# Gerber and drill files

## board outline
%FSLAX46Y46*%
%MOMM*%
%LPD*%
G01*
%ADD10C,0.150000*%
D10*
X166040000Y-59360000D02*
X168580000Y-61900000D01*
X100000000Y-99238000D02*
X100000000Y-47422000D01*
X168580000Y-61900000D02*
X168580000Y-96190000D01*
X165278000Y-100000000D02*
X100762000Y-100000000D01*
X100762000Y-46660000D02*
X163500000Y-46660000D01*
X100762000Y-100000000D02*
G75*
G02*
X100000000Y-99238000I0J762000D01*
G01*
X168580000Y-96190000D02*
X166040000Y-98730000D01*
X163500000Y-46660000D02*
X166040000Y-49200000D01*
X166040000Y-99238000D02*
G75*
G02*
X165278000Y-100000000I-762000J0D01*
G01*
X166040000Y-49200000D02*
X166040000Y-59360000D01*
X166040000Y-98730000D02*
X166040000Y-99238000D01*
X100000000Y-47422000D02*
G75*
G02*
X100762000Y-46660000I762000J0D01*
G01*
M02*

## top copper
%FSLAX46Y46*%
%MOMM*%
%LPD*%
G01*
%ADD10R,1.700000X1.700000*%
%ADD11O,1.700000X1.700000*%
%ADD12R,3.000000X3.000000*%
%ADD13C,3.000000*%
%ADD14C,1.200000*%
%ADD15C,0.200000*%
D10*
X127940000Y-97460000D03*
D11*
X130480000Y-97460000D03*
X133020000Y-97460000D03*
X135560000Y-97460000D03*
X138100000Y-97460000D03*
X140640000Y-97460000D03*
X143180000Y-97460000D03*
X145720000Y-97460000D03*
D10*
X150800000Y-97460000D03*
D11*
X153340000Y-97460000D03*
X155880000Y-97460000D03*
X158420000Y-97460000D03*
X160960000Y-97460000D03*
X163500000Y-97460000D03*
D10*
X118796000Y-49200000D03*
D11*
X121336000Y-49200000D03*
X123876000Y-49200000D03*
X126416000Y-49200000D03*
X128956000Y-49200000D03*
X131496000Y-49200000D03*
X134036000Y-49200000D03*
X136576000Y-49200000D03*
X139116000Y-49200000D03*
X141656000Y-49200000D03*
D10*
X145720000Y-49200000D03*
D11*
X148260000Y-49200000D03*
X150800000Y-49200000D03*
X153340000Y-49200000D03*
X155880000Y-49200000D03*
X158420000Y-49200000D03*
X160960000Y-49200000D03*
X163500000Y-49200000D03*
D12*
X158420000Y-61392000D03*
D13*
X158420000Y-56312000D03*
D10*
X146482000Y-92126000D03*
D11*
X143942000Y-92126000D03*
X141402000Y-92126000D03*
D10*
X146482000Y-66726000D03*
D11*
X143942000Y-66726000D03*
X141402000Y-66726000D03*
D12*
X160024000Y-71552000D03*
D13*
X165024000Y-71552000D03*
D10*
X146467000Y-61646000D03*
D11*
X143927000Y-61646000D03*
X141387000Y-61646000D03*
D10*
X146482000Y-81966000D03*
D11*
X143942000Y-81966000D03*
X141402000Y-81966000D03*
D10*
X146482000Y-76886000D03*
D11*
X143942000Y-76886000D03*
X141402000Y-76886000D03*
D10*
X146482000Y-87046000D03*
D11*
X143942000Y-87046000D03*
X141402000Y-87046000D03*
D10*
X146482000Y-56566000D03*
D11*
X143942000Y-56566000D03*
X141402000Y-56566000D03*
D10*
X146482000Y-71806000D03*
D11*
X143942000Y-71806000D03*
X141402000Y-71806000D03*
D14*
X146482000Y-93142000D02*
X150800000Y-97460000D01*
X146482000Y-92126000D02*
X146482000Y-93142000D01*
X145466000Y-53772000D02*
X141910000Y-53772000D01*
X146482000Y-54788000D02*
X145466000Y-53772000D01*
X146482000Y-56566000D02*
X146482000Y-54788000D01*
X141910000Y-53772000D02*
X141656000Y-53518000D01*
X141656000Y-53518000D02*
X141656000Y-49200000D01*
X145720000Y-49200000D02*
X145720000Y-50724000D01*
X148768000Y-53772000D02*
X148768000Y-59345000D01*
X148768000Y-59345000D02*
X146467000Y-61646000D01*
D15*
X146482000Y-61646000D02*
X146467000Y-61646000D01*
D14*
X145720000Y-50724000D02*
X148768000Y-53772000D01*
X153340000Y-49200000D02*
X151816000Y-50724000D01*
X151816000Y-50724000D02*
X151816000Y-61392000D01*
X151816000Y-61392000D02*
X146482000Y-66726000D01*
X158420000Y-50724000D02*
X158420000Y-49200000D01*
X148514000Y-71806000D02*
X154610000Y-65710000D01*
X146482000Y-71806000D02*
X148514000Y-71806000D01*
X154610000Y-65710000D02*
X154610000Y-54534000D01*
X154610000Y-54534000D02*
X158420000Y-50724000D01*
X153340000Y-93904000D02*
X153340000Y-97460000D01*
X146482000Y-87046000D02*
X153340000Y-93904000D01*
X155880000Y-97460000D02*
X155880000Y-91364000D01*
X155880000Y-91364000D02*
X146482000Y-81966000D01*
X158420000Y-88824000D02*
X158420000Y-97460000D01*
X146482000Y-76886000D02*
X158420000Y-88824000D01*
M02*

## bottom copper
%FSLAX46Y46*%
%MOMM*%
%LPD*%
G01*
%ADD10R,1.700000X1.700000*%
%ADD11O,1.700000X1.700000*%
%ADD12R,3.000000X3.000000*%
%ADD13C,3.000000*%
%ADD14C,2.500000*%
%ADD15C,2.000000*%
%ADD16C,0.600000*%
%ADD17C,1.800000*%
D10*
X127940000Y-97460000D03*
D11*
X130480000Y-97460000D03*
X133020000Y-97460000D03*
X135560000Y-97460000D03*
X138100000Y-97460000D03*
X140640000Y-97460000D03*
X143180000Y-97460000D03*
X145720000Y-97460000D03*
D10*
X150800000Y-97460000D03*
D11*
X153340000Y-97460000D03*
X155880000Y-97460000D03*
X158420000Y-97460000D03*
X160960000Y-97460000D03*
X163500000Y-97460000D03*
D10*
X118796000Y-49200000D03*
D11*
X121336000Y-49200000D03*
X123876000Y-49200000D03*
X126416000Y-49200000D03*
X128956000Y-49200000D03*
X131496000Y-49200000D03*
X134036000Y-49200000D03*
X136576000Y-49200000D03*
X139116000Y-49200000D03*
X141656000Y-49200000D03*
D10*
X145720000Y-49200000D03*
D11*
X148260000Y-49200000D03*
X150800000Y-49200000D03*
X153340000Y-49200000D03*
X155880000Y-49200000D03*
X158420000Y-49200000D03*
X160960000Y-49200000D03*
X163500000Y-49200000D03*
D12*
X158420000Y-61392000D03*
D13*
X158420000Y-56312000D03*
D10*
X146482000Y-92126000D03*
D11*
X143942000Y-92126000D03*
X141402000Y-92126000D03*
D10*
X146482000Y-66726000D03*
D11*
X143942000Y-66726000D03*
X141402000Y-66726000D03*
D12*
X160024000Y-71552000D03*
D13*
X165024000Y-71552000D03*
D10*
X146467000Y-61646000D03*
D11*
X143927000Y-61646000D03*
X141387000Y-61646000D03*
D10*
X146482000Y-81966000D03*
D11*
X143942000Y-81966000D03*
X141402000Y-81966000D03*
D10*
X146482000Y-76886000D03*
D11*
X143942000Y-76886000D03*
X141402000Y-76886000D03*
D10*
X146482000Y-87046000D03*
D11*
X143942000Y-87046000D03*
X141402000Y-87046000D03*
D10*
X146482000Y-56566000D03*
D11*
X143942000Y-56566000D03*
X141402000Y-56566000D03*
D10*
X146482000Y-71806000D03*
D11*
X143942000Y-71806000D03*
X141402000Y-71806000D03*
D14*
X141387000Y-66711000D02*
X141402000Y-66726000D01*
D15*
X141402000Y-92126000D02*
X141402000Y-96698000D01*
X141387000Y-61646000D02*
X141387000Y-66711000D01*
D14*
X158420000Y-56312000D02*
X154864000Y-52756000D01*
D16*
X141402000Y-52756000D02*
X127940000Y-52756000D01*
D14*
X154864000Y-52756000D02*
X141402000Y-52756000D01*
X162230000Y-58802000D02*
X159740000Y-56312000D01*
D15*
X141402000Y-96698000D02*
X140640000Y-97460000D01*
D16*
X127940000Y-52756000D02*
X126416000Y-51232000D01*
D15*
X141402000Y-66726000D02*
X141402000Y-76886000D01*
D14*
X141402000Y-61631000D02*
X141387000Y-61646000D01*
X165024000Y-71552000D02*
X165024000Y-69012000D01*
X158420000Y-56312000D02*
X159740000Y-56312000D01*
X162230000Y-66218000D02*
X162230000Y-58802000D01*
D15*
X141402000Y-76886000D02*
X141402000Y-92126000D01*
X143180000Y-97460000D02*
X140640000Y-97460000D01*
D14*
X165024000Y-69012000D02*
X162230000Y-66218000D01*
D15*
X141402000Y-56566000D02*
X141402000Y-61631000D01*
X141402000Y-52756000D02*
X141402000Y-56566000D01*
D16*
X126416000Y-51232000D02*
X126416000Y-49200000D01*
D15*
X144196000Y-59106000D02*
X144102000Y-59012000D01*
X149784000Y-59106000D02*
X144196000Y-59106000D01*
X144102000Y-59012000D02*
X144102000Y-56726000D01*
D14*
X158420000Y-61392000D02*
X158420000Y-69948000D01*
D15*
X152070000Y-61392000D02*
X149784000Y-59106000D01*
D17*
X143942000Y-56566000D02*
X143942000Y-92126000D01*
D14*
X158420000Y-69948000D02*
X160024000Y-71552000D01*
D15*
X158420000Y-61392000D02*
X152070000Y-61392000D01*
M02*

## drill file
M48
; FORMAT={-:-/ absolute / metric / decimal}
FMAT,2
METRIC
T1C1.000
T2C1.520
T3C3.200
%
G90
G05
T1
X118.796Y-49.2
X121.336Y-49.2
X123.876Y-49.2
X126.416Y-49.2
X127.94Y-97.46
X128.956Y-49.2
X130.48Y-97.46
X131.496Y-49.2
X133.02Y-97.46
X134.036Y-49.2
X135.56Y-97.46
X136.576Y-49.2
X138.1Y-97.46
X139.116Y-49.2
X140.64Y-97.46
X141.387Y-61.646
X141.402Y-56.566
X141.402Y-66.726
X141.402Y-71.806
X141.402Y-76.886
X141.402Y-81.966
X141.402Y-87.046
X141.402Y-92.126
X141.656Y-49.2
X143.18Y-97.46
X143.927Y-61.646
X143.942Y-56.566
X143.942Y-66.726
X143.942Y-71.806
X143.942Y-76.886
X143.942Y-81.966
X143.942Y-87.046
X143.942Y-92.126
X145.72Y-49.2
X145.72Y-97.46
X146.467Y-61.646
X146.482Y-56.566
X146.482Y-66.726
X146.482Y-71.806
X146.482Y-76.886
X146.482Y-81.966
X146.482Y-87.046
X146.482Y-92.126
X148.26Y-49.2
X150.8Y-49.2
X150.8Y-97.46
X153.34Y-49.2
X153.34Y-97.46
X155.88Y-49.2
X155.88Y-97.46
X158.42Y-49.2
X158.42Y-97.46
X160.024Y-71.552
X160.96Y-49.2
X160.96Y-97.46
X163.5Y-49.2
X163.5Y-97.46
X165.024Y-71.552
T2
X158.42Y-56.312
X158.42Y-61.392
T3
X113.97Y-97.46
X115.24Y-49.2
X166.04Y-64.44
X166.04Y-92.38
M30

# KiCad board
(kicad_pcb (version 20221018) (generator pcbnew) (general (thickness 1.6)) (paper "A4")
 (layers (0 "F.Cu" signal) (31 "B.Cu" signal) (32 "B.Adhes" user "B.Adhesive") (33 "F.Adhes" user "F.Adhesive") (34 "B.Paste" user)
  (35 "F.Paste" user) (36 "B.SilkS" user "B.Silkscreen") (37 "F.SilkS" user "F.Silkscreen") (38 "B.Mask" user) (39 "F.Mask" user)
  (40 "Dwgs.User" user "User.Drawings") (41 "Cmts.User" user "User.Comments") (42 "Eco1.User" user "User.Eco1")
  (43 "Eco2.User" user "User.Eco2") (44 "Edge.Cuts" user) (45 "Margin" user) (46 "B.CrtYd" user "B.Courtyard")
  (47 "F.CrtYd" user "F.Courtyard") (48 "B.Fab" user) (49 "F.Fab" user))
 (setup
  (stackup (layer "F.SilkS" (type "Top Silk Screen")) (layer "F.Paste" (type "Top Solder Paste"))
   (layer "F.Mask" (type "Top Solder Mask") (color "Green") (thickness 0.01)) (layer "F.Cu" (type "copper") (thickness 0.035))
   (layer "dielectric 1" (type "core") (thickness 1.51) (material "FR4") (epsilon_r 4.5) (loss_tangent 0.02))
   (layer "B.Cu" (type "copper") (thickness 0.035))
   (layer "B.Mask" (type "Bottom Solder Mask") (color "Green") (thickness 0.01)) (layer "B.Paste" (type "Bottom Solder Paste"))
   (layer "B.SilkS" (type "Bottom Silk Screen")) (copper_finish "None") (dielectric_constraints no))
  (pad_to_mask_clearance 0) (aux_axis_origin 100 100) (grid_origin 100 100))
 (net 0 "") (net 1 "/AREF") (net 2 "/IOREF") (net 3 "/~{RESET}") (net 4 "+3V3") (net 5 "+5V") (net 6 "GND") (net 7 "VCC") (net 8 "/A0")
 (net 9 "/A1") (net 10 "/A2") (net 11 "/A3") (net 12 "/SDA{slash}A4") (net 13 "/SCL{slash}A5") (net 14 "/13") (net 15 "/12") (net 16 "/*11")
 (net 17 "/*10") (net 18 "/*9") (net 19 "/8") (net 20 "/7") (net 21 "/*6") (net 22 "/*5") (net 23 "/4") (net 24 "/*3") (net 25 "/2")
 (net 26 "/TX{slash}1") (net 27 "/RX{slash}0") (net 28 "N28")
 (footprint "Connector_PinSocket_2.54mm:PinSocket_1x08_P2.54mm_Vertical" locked (layer "F.Cu") (at 127.94 97.46 90)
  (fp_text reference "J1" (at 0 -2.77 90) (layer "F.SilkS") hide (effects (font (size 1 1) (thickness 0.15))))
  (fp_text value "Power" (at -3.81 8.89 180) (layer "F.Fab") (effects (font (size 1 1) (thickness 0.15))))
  (pad "1" thru_hole rect locked (at 0 0 90) (size 1.7 1.7) (drill 1) (layers "*.Cu" "*.Mask") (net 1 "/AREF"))
  (pad "2" thru_hole oval locked (at 0 2.54 90) (size 1.7 1.7) (drill 1) (layers "*.Cu" "*.Mask") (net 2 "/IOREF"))
  (pad "3" thru_hole oval locked (at 0 5.08 90) (size 1.7 1.7) (drill 1) (layers "*.Cu" "*.Mask") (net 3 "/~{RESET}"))
  (pad "4" thru_hole oval locked (at 0 7.62 90) (size 1.7 1.7) (drill 1) (layers "*.Cu" "*.Mask") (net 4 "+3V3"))
  (pad "5" thru_hole oval locked (at 0 10.16 90) (size 1.7 1.7) (drill 1) (layers "*.Cu" "*.Mask") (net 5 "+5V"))
  (pad "6" thru_hole oval locked (at 0 12.7 90) (size 1.7 1.7) (drill 1) (layers "*.Cu" "*.Mask") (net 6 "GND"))
  (pad "7" thru_hole oval locked (at 0 15.24 90) (size 1.7 1.7) (drill 1) (layers "*.Cu" "*.Mask") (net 6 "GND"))
  (pad "8" thru_hole oval locked (at 0 17.78 90) (size 1.7 1.7) (drill 1) (layers "*.Cu" "*.Mask") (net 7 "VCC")))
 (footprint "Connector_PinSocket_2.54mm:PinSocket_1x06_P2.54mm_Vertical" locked (layer "F.Cu") (at 150.8 97.46 90)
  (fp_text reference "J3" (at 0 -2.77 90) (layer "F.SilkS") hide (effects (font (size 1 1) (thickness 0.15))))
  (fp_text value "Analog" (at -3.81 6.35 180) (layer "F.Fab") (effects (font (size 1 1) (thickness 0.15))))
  (pad "1" thru_hole rect locked (at 0 0 90) (size 1.7 1.7) (drill 1) (layers "*.Cu" "*.Mask") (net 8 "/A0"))
  (pad "2" thru_hole oval locked (at 0 2.54 90) (size 1.7 1.7) (drill 1) (layers "*.Cu" "*.Mask") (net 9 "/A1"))
  (pad "3" thru_hole oval locked (at 0 5.08 90) (size 1.7 1.7) (drill 1) (layers "*.Cu" "*.Mask") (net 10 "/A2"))
  (pad "4" thru_hole oval locked (at 0 7.62 90) (size 1.7 1.7) (drill 1) (layers "*.Cu" "*.Mask") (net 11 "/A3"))
  (pad "5" thru_hole oval locked (at 0 10.16 90) (size 1.7 1.7) (drill 1) (layers "*.Cu" "*.Mask") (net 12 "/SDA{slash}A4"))
  (pad "6" thru_hole oval locked (at 0 12.7 90) (size 1.7 1.7) (drill 1) (layers "*.Cu" "*.Mask") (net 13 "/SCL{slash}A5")))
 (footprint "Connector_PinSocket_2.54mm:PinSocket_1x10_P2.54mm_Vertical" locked (layer "F.Cu") (at 118.796 49.2 90)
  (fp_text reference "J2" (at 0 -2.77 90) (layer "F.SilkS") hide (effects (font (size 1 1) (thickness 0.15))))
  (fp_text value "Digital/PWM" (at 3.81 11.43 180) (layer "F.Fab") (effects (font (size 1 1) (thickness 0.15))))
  (pad "1" thru_hole rect locked (at 0 0 90) (size 1.7 1.7) (drill 1) (layers "*.Cu" "*.Mask") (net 13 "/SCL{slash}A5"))
  (pad "2" thru_hole oval locked (at 0 2.54 90) (size 1.7 1.7) (drill 1) (layers "*.Cu" "*.Mask") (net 12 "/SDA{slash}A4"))
  (pad "3" thru_hole oval locked (at 0 5.08 90) (size 1.7 1.7) (drill 1) (layers "*.Cu" "*.Mask") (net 1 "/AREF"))
  (pad "4" thru_hole oval locked (at 0 7.62 90) (size 1.7 1.7) (drill 1) (layers "*.Cu" "*.Mask") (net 6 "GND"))
  (pad "5" thru_hole oval locked (at 0 10.16 90) (size 1.7 1.7) (drill 1) (layers "*.Cu" "*.Mask") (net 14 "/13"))
  (pad "6" thru_hole oval locked (at 0 12.7 90) (size 1.7 1.7) (drill 1) (layers "*.Cu" "*.Mask") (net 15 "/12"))
  (pad "7" thru_hole oval locked (at 0 15.24 90) (size 1.7 1.7) (drill 1) (layers "*.Cu" "*.Mask") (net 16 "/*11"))
  (pad "8" thru_hole oval locked (at 0 17.78 90) (size 1.7 1.7) (drill 1) (layers "*.Cu" "*.Mask") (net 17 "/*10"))
  (pad "9" thru_hole oval locked (at 0 20.32 90) (size 1.7 1.7) (drill 1) (layers "*.Cu" "*.Mask") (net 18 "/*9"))
  (pad "10" thru_hole oval locked (at 0 22.86 90) (size 1.7 1.7) (drill 1) (layers "*.Cu" "*.Mask") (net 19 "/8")))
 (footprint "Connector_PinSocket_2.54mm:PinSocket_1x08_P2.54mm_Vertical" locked (layer "F.Cu") (at 145.72 49.2 90)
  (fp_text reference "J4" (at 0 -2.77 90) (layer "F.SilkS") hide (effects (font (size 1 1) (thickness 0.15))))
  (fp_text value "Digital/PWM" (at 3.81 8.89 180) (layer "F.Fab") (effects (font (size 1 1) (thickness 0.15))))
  (pad "1" thru_hole rect locked (at 0 0 90) (size 1.7 1.7) (drill 1) (layers "*.Cu" "*.Mask") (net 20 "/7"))
  (pad "2" thru_hole oval locked (at 0 2.54 90) (size 1.7 1.7) (drill 1) (layers "*.Cu" "*.Mask") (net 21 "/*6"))
  (pad "3" thru_hole oval locked (at 0 5.08 90) (size 1.7 1.7) (drill 1) (layers "*.Cu" "*.Mask") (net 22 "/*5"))
  (pad "4" thru_hole oval locked (at 0 7.62 90) (size 1.7 1.7) (drill 1) (layers "*.Cu" "*.Mask") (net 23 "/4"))
  (pad "5" thru_hole oval locked (at 0 10.16 90) (size 1.7 1.7) (drill 1) (layers "*.Cu" "*.Mask") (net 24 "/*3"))
  (pad "6" thru_hole oval locked (at 0 12.7 90) (size 1.7 1.7) (drill 1) (layers "*.Cu" "*.Mask") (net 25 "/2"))
  (pad "7" thru_hole oval locked (at 0 15.24 90) (size 1.7 1.7) (drill 1) (layers "*.Cu" "*.Mask") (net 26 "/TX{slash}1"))
  (pad "8" thru_hole oval locked (at 0 17.78 90) (size 1.7 1.7) (drill 1) (layers "*.Cu" "*.Mask") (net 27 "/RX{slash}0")))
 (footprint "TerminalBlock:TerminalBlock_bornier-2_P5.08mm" (layer "F.Cu") (at 158.42 61.392 90)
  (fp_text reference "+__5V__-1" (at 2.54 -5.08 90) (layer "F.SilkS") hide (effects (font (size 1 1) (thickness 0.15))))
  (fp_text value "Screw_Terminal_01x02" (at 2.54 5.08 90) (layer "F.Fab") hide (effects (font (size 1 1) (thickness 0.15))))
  (pad "1" thru_hole rect (at 0 0 90) (size 3 3) (drill 1.52) (layers "*.Cu" "*.Mask") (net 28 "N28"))
  (pad "2" thru_hole circle (at 5.08 0 90) (size 3 3) (drill 1.52) (layers "*.Cu" "*.Mask") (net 6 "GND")))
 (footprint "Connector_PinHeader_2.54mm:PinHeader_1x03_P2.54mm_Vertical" (layer "F.Cu") (at 146.482 92.126 -90)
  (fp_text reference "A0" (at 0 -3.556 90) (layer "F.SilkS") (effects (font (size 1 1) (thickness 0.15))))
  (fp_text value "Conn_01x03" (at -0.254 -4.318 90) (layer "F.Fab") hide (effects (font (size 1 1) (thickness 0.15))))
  (pad "1" thru_hole rect (at 0 0 270) (size 1.7 1.7) (drill 1) (layers "*.Cu" "*.Mask") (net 8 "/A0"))
  (pad "2" thru_hole oval (at 0 2.54 270) (size 1.7 1.7) (drill 1) (layers "*.Cu" "*.Mask") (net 28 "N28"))
  (pad "3" thru_hole oval (at 0 5.08 270) (size 1.7 1.7) (drill 1) (layers "*.Cu" "*.Mask") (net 6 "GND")))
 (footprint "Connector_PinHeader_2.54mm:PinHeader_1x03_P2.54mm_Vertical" (layer "F.Cu") (at 146.482 66.726 -90)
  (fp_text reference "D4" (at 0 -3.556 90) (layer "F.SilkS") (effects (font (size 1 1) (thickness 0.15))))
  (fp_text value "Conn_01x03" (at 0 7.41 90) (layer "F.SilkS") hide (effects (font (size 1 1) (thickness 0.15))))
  (pad "1" thru_hole rect (at 0 0 270) (size 1.7 1.7) (drill 1) (layers "*.Cu" "*.Mask") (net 23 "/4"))
  (pad "2" thru_hole oval (at 0 2.54 270) (size 1.7 1.7) (drill 1) (layers "*.Cu" "*.Mask") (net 28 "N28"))
  (pad "3" thru_hole oval (at 0 5.08 270) (size 1.7 1.7) (drill 1) (layers "*.Cu" "*.Mask") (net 6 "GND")))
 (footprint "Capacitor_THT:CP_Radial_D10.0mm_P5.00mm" (layer "F.Cu") (at 160.024 71.552)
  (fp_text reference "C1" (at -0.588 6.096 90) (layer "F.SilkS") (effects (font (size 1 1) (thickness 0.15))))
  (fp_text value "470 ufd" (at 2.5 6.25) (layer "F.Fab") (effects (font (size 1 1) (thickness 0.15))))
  (pad "1" thru_hole rect (at 0 0) (size 3 3) (drill 1) (layers "*.Cu" "*.Mask") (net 28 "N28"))
  (pad "2" thru_hole circle (at 5 0) (size 3 3) (drill 1) (layers "*.Cu" "*.Mask") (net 6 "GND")))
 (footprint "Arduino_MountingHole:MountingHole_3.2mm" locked (layer "F.Cu") (at 115.24 49.2)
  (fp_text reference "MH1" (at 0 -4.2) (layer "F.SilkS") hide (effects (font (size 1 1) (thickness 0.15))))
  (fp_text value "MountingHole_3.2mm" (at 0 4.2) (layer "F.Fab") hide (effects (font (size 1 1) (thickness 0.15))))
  (pad "" np_thru_hole circle locked (at 0 0) (size 3.2 3.2) (drill 3.2) (layers "*.Cu" "*.Mask")))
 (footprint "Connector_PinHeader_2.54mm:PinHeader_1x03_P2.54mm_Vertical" (layer "F.Cu") (at 146.467 61.646 -90)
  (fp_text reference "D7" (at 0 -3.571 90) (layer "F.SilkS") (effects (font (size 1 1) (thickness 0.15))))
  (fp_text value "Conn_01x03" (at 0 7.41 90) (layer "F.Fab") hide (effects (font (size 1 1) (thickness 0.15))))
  (pad "1" thru_hole rect (at 0 0 270) (size 1.7 1.7) (drill 1) (layers "*.Cu" "*.Mask") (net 20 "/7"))
  (pad "2" thru_hole oval (at 0 2.54 270) (size 1.7 1.7) (drill 1) (layers "*.Cu" "*.Mask") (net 28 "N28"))
  (pad "3" thru_hole oval (at 0 5.08 270) (size 1.7 1.7) (drill 1) (layers "*.Cu" "*.Mask") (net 6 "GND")))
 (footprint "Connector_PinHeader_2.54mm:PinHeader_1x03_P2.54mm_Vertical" (layer "F.Cu") (at 146.482 81.966 -90)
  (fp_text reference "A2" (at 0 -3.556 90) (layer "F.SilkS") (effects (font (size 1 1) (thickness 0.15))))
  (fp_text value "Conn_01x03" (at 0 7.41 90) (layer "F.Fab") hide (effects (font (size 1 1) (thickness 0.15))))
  (pad "1" thru_hole rect (at 0 0 270) (size 1.7 1.7) (drill 1) (layers "*.Cu" "*.Mask") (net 10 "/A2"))
  (pad "2" thru_hole oval (at 0 2.54 270) (size 1.7 1.7) (drill 1) (layers "*.Cu" "*.Mask") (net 28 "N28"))
  (pad "3" thru_hole oval (at 0 5.08 270) (size 1.7 1.7) (drill 1) (layers "*.Cu" "*.Mask") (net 6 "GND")))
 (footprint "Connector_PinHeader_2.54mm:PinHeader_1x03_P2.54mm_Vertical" (layer "F.Cu") (at 146.482 76.886 -90)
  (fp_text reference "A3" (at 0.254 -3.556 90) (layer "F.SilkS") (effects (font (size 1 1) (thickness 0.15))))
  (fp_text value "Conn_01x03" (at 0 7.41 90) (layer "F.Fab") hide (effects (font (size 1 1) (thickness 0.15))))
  (pad "1" thru_hole rect (at 0 0 270) (size 1.7 1.7) (drill 1) (layers "*.Cu" "*.Mask") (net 11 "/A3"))
  (pad "2" thru_hole oval (at 0 2.54 270) (size 1.7 1.7) (drill 1) (layers "*.Cu" "*.Mask") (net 28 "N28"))
  (pad "3" thru_hole oval (at 0 5.08 270) (size 1.7 1.7) (drill 1) (layers "*.Cu" "*.Mask") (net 6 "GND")))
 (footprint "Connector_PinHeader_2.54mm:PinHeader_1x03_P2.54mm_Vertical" (layer "F.Cu") (at 146.482 87.046 -90)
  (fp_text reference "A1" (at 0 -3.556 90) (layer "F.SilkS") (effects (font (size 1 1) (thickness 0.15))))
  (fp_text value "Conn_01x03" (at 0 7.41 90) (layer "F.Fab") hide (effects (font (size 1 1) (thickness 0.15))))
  (pad "1" thru_hole rect (at 0 0 270) (size 1.7 1.7) (drill 1) (layers "*.Cu" "*.Mask") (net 9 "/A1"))
  (pad "2" thru_hole oval (at 0 2.54 270) (size 1.7 1.7) (drill 1) (layers "*.Cu" "*.Mask") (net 28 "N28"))
  (pad "3" thru_hole oval (at 0 5.08 270) (size 1.7 1.7) (drill 1) (layers "*.Cu" "*.Mask") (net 6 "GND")))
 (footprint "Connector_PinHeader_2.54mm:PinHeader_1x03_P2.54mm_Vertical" (layer "F.Cu") (at 146.482 56.566 -90)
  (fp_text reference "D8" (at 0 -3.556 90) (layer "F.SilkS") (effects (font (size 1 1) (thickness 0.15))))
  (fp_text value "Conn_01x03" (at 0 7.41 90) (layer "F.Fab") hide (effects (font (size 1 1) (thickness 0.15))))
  (pad "1" thru_hole rect (at 0 0 270) (size 1.7 1.7) (drill 1) (layers "*.Cu" "*.Mask") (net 19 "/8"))
  (pad "2" thru_hole oval (at 0 2.54 270) (size 1.7 1.7) (drill 1) (layers "*.Cu" "*.Mask") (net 28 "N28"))
  (pad "3" thru_hole oval (at 0 5.08 270) (size 1.7 1.7) (drill 1) (layers "*.Cu" "*.Mask") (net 6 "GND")))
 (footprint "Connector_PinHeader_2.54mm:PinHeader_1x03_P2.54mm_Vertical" (layer "F.Cu") (at 146.482 71.806 -90)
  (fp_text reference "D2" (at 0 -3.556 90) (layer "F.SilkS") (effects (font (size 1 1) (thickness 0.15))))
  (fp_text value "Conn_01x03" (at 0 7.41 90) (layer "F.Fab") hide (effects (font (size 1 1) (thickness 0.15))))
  (pad "1" thru_hole rect (at 0 0 270) (size 1.7 1.7) (drill 1) (layers "*.Cu" "*.Mask") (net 25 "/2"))
  (pad "2" thru_hole oval (at 0 2.54 270) (size 1.7 1.7) (drill 1) (layers "*.Cu" "*.Mask") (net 28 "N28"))
  (pad "3" thru_hole oval (at 0 5.08 270) (size 1.7 1.7) (drill 1) (layers "*.Cu" "*.Mask") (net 6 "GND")))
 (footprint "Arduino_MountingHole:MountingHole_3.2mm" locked (layer "F.Cu") (at 113.97 97.46)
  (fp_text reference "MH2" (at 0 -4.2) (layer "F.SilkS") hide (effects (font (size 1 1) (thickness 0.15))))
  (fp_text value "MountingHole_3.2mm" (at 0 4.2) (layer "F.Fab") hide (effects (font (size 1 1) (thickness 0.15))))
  (pad "" np_thru_hole circle locked (at 0 0) (size 3.2 3.2) (drill 3.2) (layers "*.Cu" "*.Mask")))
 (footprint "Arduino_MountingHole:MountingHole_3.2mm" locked (layer "F.Cu") (at 166.04 64.44)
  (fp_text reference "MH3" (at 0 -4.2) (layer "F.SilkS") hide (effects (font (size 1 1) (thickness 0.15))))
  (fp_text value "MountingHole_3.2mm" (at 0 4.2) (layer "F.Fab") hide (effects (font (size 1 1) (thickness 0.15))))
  (pad "" np_thru_hole circle locked (at 0 0) (size 3.2 3.2) (drill 3.2) (layers "*.Cu" "*.Mask")))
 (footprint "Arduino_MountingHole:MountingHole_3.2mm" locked (layer "F.Cu") (at 166.04 92.38)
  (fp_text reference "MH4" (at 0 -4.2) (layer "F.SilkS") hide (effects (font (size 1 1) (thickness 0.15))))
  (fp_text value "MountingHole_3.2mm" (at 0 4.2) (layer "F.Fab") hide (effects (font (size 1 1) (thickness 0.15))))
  (pad "" np_thru_hole circle locked (at 0 0) (size 3.2 3.2) (drill 3.2) (layers "*.Cu" "*.Mask")))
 (gr_line (start 166.04 59.36) (end 168.58 61.9) (stroke (width 0.15) (type solid)) (layer "Edge.Cuts"))
 (gr_line (start 100 99.238) (end 100 47.422) (stroke (width 0.15) (type solid)) (layer "Edge.Cuts"))
 (gr_line (start 168.58 61.9) (end 168.58 96.19) (stroke (width 0.15) (type solid)) (layer "Edge.Cuts"))
 (gr_line (start 165.278 100) (end 100.762 100) (stroke (width 0.15) (type solid)) (layer "Edge.Cuts"))
 (gr_line (start 100.762 46.66) (end 163.5 46.66) (stroke (width 0.15) (type solid)) (layer "Edge.Cuts"))
 (gr_arc (start 100.762 100) (mid 100.223185 99.776815) (end 100 99.238) (stroke (width 0.15) (type solid)) (layer "Edge.Cuts"))
 (gr_line (start 168.58 96.19) (end 166.04 98.73) (stroke (width 0.15) (type solid)) (layer "Edge.Cuts"))
 (gr_line (start 163.5 46.66) (end 166.04 49.2) (stroke (width 0.15) (type solid)) (layer "Edge.Cuts"))
 (gr_arc (start 166.04 99.238) (mid 165.816815 99.776815) (end 165.278 100) (stroke (width 0.15) (type solid)) (layer "Edge.Cuts"))
 (gr_line (start 166.04 49.2) (end 166.04 59.36) (stroke (width 0.15) (type solid)) (layer "Edge.Cuts"))
 (gr_line (start 166.04 98.73) (end 166.04 99.238) (stroke (width 0.15) (type solid)) (layer "Edge.Cuts"))
 (gr_arc (start 100 47.422) (mid 100.223185 46.883185) (end 100.762 46.66) (stroke (width 0.15) (type solid)) (layer "Edge.Cuts"))
 (segment (start 141.387 66.711) (end 141.402 66.726) (width 2.5) (layer "B.Cu") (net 6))
 (segment (start 141.402 92.126) (end 141.402 96.698) (width 2) (layer "B.Cu") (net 6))
 (segment (start 141.387 61.646) (end 141.387 66.711) (width 2) (layer "B.Cu") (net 6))
 (segment (start 158.42 56.312) (end 154.864 52.756) (width 2.5) (layer "B.Cu") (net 6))
 (segment (start 141.402 52.756) (end 127.94 52.756) (width 0.6) (layer "B.Cu") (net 6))
 (segment (start 154.864 52.756) (end 141.402 52.756) (width 2.5) (layer "B.Cu") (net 6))
 (segment (start 162.23 58.802) (end 159.74 56.312) (width 2.5) (layer "B.Cu") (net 6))
 (segment (start 141.402 96.698) (end 140.64 97.46) (width 2) (layer "B.Cu") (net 6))
 (segment (start 127.94 52.756) (end 126.416 51.232) (width 0.6) (layer "B.Cu") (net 6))
 (segment (start 141.402 66.726) (end 141.402 76.886) (width 2) (layer "B.Cu") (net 6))
 (segment (start 141.402 61.631) (end 141.387 61.646) (width 2.5) (layer "B.Cu") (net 6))
 (segment (start 165.024 71.552) (end 165.024 69.012) (width 2.5) (layer "B.Cu") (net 6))
 (segment (start 158.42 56.312) (end 159.74 56.312) (width 2.5) (layer "B.Cu") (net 6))
 (segment (start 162.23 66.218) (end 162.23 58.802) (width 2.5) (layer "B.Cu") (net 6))
 (segment (start 141.402 76.886) (end 141.402 92.126) (width 2) (layer "B.Cu") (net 6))
 (segment (start 143.18 97.46) (end 140.64 97.46) (width 2) (layer "B.Cu") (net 6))
 (segment (start 165.024 69.012) (end 162.23 66.218) (width 2.5) (layer "B.Cu") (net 6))
 (segment (start 141.402 56.566) (end 141.402 61.631) (width 2) (layer "B.Cu") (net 6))
 (segment (start 141.402 52.756) (end 141.402 56.566) (width 2) (layer "B.Cu") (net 6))
 (segment (start 126.416 51.232) (end 126.416 49.2) (width 0.6) (layer "B.Cu") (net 6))
 (segment (start 146.482 93.142) (end 150.8 97.46) (width 1.2) (layer "F.Cu") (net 8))
 (segment (start 146.482 92.126) (end 146.482 93.142) (width 1.2) (layer "F.Cu") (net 8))
 (segment (start 145.466 53.772) (end 141.91 53.772) (width 1.2) (layer "F.Cu") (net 19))
 (segment (start 146.482 54.788) (end 145.466 53.772) (width 1.2) (layer "F.Cu") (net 19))
 (segment (start 146.482 56.566) (end 146.482 54.788) (width 1.2) (layer "F.Cu") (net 19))
 (segment (start 141.91 53.772) (end 141.656 53.518) (width 1.2) (layer "F.Cu") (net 19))
 (segment (start 141.656 53.518) (end 141.656 49.2) (width 1.2) (layer "F.Cu") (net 19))
 (segment (start 145.72 49.2) (end 145.72 50.724) (width 1.2) (layer "F.Cu") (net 20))
 (segment (start 148.768 53.772) (end 148.768 59.345) (width 1.2) (layer "F.Cu") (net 20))
 (segment (start 148.768 59.345) (end 146.467 61.646) (width 1.2) (layer "F.Cu") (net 20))
 (segment (start 146.482 61.646) (end 146.467 61.646) (width 0.2) (layer "F.Cu") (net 20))
 (segment (start 145.72 50.724) (end 148.768 53.772) (width 1.2) (layer "F.Cu") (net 20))
 (segment (start 153.34 49.2) (end 151.816 50.724) (width 1.2) (layer "F.Cu") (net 23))
 (segment (start 151.816 50.724) (end 151.816 61.392) (width 1.2) (layer "F.Cu") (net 23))
 (segment (start 151.816 61.392) (end 146.482 66.726) (width 1.2) (layer "F.Cu") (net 23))
 (segment (start 158.42 50.724) (end 158.42 49.2) (width 1.2) (layer "F.Cu") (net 25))
 (segment (start 148.514 71.806) (end 154.61 65.71) (width 1.2) (layer "F.Cu") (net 25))
 (segment (start 146.482 71.806) (end 148.514 71.806) (width 1.2) (layer "F.Cu") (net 25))
 (segment (start 154.61 65.71) (end 154.61 54.534) (width 1.2) (layer "F.Cu") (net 25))
 (segment (start 154.61 54.534) (end 158.42 50.724) (width 1.2) (layer "F.Cu") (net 25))
 (segment (start 153.34 93.904) (end 153.34 97.46) (width 1.2) (layer "F.Cu") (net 9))
 (segment (start 146.482 87.046) (end 153.34 93.904) (width 1.2) (layer "F.Cu") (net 9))
 (segment (start 155.88 97.46) (end 155.88 91.364) (width 1.2) (layer "F.Cu") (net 10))
 (segment (start 155.88 91.364) (end 146.482 81.966) (width 1.2) (layer "F.Cu") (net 10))
 (segment (start 158.42 88.824) (end 158.42 97.46) (width 1.2) (layer "F.Cu") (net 11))
 (segment (start 146.482 76.886) (end 158.42 88.824) (width 1.2) (layer "F.Cu") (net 11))
 (segment (start 144.196 59.106) (end 144.102 59.012) (width 2) (layer "B.Cu") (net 28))
 (segment (start 149.784 59.106) (end 144.196 59.106) (width 2) (layer "B.Cu") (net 28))
 (segment (start 144.102 59.012) (end 144.102 56.726) (width 2) (layer "B.Cu") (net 28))
 (segment (start 158.42 61.392) (end 158.42 69.948) (width 2.5) (layer "B.Cu") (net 28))
 (segment (start 152.07 61.392) (end 149.784 59.106) (width 2) (layer "B.Cu") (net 28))
 (segment (start 143.942 56.566) (end 143.942 92.126) (width 1.8) (layer "B.Cu") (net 28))
 (segment (start 158.42 69.948) (end 160.024 71.552) (width 2.5) (layer "B.Cu") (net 28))
 (segment (start 158.42 61.392) (end 152.07 61.392) (width 2) (layer "B.Cu") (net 28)))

